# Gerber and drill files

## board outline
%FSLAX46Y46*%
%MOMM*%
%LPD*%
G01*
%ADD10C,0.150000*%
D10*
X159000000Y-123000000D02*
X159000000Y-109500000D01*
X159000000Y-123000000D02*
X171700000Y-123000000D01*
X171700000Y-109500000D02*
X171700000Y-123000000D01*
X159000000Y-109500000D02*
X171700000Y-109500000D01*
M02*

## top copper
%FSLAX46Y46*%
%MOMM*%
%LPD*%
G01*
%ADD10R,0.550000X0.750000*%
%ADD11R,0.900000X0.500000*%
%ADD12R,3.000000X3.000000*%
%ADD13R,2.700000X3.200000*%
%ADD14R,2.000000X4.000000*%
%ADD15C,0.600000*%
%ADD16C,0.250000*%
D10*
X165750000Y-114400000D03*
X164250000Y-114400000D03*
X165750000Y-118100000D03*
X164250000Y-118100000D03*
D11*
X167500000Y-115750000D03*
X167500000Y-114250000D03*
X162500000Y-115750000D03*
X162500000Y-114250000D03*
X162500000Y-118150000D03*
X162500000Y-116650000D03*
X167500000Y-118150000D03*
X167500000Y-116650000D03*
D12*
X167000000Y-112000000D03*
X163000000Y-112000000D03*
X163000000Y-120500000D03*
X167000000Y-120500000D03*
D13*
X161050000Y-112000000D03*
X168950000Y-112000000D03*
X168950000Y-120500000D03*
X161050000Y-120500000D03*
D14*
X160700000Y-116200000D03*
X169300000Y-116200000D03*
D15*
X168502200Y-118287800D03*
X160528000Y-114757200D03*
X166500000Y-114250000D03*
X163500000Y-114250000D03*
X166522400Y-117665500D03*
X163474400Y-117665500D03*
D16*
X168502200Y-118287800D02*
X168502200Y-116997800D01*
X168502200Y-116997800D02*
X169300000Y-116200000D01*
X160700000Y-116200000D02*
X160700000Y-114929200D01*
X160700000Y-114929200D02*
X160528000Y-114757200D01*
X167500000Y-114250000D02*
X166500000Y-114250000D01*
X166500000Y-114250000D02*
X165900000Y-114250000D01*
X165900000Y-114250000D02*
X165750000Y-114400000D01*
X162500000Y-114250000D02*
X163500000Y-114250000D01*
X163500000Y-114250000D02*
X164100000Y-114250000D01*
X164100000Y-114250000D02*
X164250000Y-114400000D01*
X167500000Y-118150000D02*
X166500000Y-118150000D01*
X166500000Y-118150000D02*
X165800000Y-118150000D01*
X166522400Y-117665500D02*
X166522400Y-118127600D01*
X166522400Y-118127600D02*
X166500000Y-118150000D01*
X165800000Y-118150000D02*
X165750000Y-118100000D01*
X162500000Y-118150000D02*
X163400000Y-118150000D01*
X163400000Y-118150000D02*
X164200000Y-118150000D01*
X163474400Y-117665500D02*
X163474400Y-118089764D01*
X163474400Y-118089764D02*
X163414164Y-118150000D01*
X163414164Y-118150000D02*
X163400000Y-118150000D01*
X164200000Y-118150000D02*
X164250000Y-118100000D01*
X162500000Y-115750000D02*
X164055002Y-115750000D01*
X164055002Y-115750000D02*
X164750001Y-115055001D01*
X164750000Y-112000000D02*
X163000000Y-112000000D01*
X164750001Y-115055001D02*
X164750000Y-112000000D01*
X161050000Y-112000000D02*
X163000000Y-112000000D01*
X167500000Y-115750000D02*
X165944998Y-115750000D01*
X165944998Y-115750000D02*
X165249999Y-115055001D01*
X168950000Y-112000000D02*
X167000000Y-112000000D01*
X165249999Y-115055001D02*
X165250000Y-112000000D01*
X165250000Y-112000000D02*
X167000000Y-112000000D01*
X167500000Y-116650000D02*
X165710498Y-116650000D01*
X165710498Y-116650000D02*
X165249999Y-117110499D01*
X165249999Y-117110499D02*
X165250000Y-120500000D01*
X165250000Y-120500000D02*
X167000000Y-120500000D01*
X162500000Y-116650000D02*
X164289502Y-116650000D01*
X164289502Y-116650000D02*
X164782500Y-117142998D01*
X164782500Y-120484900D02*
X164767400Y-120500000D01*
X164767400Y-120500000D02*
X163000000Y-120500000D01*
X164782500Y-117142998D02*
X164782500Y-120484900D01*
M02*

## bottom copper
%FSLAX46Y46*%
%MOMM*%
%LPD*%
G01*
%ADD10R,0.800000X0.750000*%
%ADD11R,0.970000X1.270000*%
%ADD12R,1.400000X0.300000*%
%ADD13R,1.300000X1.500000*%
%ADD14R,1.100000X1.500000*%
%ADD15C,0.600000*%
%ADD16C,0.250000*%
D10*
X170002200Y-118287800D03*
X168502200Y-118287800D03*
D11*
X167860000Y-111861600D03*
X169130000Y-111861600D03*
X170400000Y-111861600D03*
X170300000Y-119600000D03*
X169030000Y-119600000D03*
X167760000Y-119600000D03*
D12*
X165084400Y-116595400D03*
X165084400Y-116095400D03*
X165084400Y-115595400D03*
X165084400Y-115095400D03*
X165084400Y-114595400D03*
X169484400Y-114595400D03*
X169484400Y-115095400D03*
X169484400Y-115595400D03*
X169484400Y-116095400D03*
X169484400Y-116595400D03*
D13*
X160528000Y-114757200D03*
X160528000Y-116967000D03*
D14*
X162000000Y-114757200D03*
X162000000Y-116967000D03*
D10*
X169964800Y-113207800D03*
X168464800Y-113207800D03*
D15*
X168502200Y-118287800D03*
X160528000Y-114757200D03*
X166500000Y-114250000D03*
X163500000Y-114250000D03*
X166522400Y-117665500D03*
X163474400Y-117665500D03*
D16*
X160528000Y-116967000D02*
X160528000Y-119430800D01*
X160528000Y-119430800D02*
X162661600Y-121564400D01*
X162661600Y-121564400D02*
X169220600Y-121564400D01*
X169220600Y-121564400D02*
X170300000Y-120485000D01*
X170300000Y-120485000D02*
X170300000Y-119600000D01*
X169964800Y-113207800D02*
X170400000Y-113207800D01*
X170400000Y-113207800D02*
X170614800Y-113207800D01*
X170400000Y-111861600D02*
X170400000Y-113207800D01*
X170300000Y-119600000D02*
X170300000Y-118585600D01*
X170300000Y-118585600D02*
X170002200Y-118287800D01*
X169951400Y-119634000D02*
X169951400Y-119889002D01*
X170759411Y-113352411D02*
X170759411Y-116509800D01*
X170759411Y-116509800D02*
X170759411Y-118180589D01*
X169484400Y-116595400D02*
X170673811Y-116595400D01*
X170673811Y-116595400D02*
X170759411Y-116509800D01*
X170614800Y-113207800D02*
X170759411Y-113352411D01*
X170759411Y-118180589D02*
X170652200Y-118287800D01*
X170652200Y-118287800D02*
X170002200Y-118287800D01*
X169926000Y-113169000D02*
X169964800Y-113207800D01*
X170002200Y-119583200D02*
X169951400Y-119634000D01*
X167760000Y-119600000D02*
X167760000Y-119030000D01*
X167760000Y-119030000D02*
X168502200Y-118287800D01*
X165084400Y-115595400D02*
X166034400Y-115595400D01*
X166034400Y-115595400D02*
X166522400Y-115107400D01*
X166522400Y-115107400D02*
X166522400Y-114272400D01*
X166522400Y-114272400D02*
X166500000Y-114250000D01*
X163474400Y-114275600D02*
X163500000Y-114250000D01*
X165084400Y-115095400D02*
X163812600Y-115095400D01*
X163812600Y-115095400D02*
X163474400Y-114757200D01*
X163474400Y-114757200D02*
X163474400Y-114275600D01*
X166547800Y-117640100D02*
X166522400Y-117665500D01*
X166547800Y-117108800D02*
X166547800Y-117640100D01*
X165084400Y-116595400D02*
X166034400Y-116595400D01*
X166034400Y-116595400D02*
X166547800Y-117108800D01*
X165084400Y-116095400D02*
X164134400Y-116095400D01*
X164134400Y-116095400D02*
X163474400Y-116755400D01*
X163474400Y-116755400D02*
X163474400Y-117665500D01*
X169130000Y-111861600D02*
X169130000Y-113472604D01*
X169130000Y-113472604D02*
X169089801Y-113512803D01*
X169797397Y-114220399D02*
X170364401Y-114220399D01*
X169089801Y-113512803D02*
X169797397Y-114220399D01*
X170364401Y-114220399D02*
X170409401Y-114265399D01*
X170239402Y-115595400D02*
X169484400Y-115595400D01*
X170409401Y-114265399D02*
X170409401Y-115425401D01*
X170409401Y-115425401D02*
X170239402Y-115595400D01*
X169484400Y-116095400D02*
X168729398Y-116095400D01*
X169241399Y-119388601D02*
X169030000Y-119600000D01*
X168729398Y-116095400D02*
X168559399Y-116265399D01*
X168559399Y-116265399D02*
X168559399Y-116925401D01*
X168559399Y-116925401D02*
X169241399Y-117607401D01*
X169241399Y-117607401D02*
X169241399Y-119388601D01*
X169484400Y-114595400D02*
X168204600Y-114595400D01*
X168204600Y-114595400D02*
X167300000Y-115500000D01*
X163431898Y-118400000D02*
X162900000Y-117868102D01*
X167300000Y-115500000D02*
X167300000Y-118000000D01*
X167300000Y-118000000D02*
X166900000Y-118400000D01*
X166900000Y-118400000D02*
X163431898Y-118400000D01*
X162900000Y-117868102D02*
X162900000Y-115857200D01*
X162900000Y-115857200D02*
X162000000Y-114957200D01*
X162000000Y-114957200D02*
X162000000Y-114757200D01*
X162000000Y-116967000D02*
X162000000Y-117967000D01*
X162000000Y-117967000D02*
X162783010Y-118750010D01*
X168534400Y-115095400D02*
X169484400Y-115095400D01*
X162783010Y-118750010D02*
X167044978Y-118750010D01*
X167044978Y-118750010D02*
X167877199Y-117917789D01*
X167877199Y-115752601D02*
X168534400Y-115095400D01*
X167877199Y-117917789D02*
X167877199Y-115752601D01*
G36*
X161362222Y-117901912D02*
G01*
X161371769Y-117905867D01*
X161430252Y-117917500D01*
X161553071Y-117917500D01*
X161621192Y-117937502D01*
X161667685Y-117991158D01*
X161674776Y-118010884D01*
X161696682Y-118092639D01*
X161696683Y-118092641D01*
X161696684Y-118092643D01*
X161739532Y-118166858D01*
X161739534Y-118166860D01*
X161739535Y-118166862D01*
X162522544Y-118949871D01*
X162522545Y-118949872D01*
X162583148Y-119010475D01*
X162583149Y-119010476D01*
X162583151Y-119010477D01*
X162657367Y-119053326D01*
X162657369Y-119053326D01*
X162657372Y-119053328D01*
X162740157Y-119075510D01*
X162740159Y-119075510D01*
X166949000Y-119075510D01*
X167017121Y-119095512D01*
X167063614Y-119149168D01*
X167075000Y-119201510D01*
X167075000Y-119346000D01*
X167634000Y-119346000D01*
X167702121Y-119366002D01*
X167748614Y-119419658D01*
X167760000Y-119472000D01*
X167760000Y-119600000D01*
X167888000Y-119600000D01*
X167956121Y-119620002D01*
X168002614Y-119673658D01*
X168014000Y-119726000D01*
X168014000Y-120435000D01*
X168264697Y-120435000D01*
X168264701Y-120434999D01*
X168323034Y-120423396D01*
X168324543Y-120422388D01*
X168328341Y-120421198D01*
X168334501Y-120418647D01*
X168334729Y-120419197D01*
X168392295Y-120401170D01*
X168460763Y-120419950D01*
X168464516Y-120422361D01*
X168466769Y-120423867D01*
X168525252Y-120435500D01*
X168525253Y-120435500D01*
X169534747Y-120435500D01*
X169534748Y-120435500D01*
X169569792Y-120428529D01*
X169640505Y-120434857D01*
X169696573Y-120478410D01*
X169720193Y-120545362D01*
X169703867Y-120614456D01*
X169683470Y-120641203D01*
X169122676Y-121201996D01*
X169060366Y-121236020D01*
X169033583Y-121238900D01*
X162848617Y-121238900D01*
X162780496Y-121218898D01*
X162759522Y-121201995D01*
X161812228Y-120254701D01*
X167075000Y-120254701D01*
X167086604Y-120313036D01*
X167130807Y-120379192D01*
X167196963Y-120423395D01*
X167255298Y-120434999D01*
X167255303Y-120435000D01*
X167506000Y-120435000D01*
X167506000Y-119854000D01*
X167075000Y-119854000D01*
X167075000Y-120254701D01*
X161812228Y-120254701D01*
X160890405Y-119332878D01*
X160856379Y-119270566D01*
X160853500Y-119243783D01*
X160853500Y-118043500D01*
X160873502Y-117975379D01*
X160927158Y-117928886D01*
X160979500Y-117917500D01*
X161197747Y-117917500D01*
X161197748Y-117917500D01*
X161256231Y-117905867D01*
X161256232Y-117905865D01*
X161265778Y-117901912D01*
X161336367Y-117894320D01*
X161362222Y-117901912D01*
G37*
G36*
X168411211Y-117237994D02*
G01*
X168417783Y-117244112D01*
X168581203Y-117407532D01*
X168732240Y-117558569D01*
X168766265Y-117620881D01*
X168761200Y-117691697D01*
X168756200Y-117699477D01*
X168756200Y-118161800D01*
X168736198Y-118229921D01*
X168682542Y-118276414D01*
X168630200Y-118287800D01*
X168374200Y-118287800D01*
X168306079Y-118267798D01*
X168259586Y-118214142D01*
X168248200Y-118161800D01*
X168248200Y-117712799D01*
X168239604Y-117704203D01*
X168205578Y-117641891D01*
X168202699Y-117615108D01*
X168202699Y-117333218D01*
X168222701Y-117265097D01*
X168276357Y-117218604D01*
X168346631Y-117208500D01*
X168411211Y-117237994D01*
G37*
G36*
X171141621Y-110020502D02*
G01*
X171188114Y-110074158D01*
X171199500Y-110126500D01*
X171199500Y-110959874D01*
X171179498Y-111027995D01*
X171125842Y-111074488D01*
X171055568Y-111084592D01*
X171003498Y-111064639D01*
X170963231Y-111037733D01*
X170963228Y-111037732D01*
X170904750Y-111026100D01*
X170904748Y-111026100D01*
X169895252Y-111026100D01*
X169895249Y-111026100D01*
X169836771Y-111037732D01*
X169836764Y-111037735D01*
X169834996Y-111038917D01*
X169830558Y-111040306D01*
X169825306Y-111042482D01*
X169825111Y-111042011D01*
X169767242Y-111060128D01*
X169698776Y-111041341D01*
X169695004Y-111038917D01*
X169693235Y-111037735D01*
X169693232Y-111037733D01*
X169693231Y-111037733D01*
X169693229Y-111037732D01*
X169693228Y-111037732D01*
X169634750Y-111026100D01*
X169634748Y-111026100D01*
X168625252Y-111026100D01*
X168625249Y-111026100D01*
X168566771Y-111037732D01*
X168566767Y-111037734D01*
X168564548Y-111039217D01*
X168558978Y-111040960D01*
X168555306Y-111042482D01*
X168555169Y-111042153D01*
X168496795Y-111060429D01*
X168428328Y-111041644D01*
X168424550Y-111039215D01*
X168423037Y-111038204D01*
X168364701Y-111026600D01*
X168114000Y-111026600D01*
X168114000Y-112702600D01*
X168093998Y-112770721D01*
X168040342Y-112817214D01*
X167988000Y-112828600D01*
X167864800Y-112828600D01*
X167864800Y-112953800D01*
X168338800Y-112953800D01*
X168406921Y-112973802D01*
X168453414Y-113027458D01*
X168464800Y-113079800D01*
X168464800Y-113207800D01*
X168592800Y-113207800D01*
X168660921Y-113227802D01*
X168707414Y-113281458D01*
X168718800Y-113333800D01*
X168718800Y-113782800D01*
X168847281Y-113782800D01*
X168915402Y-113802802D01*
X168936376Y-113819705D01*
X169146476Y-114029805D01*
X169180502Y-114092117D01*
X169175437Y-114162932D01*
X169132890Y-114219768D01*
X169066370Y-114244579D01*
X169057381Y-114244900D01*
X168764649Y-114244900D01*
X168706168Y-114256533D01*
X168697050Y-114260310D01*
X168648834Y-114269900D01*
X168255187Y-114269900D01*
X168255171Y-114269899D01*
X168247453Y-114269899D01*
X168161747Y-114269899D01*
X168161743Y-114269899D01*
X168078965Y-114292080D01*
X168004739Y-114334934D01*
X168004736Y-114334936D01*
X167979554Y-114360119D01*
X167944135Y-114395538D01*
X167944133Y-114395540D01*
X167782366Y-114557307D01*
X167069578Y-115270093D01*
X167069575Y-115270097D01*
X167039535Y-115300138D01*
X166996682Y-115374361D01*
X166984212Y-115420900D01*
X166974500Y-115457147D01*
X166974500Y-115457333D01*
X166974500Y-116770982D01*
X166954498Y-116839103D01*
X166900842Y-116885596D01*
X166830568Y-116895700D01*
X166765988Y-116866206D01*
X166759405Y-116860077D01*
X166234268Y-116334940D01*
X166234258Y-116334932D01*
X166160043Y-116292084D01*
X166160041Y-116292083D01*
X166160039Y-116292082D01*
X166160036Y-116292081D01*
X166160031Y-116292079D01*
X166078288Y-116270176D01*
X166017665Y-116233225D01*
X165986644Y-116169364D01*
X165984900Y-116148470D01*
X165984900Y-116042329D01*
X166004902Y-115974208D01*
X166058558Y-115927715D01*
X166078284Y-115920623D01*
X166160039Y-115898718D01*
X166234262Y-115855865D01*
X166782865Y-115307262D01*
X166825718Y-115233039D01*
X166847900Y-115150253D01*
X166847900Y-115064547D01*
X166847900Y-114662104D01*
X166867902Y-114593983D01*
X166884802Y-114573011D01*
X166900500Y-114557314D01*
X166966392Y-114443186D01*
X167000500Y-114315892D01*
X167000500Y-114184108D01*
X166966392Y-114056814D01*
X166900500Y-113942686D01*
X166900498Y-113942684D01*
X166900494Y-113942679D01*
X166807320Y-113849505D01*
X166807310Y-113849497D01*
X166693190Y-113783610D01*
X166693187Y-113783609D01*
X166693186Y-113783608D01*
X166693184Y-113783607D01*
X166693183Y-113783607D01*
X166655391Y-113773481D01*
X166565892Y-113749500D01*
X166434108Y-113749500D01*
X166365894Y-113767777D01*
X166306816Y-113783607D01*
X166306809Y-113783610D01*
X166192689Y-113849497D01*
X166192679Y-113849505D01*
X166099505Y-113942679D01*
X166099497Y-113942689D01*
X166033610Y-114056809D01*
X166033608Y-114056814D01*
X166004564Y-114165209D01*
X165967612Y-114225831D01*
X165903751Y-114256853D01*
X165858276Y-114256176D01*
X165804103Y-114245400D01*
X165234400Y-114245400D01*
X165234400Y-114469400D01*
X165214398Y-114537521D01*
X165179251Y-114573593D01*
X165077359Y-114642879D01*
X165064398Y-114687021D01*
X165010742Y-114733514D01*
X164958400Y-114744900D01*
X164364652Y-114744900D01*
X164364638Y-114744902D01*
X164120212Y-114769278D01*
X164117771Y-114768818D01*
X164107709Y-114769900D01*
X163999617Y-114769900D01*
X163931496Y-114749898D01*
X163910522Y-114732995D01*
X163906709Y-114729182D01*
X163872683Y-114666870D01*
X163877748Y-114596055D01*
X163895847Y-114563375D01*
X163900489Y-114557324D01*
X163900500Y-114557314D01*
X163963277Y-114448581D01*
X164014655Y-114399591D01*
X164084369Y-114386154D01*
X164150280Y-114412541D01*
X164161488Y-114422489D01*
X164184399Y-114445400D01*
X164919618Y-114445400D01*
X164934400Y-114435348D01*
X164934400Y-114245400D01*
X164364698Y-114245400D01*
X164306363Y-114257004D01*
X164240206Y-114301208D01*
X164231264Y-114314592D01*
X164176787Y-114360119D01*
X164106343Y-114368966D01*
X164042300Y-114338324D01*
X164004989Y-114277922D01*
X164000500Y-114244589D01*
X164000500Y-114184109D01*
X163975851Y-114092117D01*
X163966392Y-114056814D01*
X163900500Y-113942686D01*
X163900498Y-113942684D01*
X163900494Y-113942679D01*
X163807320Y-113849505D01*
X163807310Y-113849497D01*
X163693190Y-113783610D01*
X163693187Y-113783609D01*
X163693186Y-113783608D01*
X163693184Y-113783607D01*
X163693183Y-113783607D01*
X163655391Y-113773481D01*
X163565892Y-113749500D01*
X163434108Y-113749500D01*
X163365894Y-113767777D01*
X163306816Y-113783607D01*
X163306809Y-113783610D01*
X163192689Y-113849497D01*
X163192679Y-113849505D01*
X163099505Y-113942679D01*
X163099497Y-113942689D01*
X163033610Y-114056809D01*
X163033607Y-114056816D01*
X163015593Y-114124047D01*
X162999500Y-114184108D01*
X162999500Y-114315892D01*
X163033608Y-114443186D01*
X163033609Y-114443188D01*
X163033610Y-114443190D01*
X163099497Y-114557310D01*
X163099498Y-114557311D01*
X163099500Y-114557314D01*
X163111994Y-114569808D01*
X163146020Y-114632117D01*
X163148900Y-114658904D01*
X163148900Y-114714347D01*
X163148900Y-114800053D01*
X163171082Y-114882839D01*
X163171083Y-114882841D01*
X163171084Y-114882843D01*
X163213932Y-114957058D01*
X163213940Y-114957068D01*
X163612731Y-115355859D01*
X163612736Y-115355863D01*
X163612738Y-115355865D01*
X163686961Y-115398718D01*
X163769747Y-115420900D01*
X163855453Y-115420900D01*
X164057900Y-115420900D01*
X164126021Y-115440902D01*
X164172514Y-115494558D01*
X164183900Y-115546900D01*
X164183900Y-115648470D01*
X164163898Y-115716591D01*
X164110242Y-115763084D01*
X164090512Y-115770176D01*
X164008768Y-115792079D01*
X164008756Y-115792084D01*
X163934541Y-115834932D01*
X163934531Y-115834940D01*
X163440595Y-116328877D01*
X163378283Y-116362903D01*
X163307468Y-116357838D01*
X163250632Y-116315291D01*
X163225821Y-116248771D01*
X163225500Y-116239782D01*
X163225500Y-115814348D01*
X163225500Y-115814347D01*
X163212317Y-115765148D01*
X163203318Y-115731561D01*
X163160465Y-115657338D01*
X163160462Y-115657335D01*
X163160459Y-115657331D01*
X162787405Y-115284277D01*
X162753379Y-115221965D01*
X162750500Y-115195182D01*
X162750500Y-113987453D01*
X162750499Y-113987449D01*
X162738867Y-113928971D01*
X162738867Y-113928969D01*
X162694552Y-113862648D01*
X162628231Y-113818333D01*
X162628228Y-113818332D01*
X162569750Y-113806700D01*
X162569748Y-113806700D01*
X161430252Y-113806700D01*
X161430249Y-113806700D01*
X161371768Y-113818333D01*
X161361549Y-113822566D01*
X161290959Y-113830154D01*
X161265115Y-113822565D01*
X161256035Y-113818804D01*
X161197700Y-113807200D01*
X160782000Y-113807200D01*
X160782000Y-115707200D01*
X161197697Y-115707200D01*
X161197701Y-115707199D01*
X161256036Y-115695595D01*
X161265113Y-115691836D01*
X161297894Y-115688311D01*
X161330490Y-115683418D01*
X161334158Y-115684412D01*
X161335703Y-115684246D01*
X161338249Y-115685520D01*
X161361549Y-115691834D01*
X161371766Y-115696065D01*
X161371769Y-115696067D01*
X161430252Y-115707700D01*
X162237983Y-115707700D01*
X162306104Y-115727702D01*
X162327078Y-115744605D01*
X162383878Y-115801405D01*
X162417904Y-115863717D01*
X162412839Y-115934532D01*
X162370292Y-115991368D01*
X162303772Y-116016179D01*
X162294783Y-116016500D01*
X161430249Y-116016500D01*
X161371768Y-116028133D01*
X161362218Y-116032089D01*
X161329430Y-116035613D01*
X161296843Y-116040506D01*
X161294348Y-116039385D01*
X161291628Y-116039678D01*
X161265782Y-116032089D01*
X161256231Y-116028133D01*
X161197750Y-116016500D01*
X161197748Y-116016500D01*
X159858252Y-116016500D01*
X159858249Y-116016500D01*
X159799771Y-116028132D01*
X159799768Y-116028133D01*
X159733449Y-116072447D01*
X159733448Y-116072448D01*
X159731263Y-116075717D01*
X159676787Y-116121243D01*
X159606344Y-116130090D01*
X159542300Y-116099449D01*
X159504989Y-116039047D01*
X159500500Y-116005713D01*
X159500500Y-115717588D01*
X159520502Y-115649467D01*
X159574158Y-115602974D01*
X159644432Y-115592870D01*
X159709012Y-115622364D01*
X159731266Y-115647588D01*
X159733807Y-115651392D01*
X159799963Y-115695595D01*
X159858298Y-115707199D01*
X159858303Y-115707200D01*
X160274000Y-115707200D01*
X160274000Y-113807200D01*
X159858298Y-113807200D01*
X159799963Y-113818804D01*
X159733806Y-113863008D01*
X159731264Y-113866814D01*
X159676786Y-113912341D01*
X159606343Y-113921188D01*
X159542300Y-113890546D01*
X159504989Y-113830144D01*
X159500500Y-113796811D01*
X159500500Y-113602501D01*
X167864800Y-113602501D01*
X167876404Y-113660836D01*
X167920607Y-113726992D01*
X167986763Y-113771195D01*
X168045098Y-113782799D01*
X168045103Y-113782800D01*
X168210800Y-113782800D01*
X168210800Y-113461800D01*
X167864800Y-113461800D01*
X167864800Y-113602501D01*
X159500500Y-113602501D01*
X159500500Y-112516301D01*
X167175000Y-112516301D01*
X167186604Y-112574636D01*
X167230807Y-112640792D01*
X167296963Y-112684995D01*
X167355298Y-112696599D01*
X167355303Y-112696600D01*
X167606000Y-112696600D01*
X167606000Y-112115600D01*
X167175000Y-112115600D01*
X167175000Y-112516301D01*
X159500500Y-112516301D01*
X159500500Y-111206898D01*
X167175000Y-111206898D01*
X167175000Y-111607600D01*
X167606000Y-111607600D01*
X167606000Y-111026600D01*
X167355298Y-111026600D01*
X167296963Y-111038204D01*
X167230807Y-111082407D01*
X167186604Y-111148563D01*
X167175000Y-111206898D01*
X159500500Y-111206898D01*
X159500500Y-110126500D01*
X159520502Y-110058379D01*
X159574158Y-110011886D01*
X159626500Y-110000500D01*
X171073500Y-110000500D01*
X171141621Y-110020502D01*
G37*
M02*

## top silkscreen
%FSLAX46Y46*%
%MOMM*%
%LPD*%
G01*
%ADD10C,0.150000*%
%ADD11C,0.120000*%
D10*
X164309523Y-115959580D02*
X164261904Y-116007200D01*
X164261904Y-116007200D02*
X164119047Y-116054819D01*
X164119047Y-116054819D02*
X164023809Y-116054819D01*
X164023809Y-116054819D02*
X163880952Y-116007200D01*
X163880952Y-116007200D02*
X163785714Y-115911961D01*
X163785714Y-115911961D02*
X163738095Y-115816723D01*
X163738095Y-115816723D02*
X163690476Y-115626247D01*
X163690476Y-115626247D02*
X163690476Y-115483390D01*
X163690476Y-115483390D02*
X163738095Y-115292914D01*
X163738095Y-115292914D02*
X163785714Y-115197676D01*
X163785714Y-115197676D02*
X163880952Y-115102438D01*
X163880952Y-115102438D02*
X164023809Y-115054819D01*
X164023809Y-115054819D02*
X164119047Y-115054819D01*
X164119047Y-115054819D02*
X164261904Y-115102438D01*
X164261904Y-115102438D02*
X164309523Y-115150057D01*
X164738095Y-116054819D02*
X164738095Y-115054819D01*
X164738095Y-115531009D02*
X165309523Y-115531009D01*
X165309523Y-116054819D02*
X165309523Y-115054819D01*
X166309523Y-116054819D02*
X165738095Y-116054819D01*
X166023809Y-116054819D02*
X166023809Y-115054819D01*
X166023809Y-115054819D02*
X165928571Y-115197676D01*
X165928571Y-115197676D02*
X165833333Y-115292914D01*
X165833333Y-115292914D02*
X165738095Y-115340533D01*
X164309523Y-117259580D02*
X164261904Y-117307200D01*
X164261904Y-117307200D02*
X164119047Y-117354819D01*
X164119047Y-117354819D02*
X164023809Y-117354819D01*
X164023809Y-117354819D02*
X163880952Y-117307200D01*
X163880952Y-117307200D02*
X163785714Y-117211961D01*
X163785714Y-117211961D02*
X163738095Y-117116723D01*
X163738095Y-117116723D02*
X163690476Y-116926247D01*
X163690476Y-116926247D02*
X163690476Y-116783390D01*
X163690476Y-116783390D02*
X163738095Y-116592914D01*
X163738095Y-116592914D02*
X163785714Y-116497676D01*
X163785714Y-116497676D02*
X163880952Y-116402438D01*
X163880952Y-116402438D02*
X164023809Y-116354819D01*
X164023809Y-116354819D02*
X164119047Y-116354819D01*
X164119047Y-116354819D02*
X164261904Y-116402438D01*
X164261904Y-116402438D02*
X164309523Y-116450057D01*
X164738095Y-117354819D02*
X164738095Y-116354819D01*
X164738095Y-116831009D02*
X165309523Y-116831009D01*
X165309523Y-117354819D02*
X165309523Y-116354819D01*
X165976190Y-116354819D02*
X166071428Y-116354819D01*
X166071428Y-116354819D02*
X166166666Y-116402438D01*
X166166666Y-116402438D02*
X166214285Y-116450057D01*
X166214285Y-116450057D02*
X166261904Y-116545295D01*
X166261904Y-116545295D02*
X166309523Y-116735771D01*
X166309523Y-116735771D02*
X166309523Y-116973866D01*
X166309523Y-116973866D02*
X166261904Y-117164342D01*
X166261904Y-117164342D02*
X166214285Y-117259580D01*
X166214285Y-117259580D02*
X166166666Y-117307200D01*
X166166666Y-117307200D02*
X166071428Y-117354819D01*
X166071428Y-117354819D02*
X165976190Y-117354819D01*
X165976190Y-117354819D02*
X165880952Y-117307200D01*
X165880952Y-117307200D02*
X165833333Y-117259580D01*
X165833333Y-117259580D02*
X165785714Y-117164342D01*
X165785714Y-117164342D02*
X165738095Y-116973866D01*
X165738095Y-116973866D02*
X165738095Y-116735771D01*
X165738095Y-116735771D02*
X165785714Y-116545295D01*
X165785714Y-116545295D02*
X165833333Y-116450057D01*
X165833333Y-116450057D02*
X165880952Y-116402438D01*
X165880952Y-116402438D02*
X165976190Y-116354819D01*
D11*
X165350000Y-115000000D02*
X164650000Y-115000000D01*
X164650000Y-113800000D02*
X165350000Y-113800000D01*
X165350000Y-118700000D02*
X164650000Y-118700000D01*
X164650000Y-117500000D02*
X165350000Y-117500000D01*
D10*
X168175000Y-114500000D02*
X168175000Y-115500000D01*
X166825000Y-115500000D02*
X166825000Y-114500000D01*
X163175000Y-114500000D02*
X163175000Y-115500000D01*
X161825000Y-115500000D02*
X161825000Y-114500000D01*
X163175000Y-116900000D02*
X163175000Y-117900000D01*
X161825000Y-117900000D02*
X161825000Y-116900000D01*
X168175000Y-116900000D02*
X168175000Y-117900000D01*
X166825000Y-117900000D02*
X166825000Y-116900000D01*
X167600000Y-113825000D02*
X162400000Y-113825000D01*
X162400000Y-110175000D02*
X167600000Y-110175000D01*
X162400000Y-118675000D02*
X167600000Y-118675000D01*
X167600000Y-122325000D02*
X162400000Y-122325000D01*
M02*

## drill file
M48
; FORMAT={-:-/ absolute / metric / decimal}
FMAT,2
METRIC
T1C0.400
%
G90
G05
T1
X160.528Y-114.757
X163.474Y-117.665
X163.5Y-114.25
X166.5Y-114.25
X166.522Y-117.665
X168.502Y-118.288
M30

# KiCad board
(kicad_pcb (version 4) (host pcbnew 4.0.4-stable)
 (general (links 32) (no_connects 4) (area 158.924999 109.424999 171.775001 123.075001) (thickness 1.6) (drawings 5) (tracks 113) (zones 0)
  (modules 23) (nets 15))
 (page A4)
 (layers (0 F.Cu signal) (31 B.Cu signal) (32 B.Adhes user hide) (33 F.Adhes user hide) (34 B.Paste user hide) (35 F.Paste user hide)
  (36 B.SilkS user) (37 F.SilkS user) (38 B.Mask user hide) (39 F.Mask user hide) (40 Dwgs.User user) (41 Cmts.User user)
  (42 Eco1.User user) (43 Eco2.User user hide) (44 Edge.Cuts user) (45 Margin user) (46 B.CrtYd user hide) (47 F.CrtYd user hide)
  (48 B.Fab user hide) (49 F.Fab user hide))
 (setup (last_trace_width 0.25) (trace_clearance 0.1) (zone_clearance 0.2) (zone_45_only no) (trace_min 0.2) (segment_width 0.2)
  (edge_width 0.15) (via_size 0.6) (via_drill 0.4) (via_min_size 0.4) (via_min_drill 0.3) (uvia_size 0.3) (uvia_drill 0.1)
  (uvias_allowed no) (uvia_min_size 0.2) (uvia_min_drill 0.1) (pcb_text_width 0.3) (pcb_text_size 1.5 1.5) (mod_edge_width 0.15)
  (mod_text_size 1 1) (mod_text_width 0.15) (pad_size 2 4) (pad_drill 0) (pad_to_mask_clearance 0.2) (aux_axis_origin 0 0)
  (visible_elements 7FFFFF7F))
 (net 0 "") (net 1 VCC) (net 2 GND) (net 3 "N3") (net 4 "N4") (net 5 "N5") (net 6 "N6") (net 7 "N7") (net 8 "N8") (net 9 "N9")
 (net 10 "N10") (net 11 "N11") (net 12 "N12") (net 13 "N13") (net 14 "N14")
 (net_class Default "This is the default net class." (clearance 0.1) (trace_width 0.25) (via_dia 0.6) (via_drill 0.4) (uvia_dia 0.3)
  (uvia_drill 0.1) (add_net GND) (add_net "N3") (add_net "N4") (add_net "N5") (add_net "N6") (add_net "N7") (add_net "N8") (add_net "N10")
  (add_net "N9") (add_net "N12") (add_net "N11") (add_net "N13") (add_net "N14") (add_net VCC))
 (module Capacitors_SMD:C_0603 (layer B.Cu) (at 169.2522 118.2878 180)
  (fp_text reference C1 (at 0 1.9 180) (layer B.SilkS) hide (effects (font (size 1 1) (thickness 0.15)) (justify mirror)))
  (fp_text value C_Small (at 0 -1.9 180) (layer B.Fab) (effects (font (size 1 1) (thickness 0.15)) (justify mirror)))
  (pad 1 smd rect (at -0.75 0 180) (size 0.8 0.75) (layers B.Cu B.Paste B.Mask) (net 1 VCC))
  (pad 2 smd rect (at 0.75 0 180) (size 0.8 0.75) (layers B.Cu B.Paste B.Mask) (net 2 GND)))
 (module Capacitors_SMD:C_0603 (layer F.Cu) (at 165 114.4 180)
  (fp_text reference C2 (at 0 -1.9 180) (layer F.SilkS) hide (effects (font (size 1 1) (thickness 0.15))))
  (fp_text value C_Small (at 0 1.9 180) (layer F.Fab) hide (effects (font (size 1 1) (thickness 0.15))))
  (fp_line (start -0.35 -0.6) (end 0.35 -0.6) (layer F.SilkS) (width 0.12))
  (fp_line (start 0.35 0.6) (end -0.35 0.6) (layer F.SilkS) (width 0.12))
  (pad 1 smd rect (at -0.75 0 180) (size 0.55 0.75) (layers F.Cu F.Paste F.Mask) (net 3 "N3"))
  (pad 2 smd rect (at 0.75 0 180) (size 0.55 0.75) (layers F.Cu F.Paste F.Mask) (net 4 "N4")))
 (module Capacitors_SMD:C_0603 (layer F.Cu) (at 165 118.1 180)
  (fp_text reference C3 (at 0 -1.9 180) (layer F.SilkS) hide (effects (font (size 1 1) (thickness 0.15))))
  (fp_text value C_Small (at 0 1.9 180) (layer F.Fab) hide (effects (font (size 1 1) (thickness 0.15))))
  (fp_line (start -0.35 -0.6) (end 0.35 -0.6) (layer F.SilkS) (width 0.12))
  (fp_line (start 0.35 0.6) (end -0.35 0.6) (layer F.SilkS) (width 0.12))
  (pad 1 smd rect (at -0.75 0 180) (size 0.55 0.75) (layers F.Cu F.Paste F.Mask) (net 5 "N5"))
  (pad 2 smd rect (at 0.75 0 180) (size 0.55 0.75) (layers F.Cu F.Paste F.Mask) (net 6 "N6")))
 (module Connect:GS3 (layer B.Cu) (at 169.13 111.8616 270)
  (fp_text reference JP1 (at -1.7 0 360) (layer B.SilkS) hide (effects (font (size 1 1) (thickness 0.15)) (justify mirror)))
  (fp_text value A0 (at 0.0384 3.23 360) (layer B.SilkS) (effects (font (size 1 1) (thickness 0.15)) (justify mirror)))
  (pad 1 smd rect (at 0 1.27 270) (size 1.27 0.97) (layers B.Cu B.Paste B.Mask) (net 2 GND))
  (pad 2 smd rect (at 0 0 270) (size 1.27 0.97) (layers B.Cu B.Paste B.Mask) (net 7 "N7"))
  (pad 3 smd rect (at 0 -1.27 270) (size 1.27 0.97) (layers B.Cu B.Paste B.Mask) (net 1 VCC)))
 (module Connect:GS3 (layer B.Cu) (at 169.03 119.6 90)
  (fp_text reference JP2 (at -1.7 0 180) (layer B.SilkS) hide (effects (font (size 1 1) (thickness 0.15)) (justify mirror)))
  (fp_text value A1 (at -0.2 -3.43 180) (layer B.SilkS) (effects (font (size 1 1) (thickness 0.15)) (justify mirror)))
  (pad 1 smd rect (at 0 1.27 90) (size 1.27 0.97) (layers B.Cu B.Paste B.Mask) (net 1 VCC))
  (pad 2 smd rect (at 0 0 90) (size 1.27 0.97) (layers B.Cu B.Paste B.Mask) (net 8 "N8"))
  (pad 3 smd rect (at 0 -1.27 90) (size 1.27 0.97) (layers B.Cu B.Paste B.Mask) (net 2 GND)))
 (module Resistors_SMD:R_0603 (layer F.Cu) (at 167.5 115 90)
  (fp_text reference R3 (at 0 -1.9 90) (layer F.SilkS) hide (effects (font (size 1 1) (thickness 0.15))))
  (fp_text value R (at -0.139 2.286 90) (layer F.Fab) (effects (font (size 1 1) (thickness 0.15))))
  (fp_line (start 0.5 0.675) (end -0.5 0.675) (layer F.SilkS) (width 0.15))
  (fp_line (start -0.5 -0.675) (end 0.5 -0.675) (layer F.SilkS) (width 0.15))
  (pad 1 smd rect (at -0.75 0 90) (size 0.5 0.9) (layers F.Cu F.Paste F.Mask) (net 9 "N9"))
  (pad 2 smd rect (at 0.75 0 90) (size 0.5 0.9) (layers F.Cu F.Paste F.Mask) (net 3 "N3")))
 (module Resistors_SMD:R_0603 (layer F.Cu) (at 162.5 115 90)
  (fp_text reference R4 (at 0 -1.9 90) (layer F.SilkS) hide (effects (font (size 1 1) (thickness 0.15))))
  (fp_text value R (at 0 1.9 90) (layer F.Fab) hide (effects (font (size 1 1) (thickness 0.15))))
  (fp_line (start 0.5 0.675) (end -0.5 0.675) (layer F.SilkS) (width 0.15))
  (fp_line (start -0.5 -0.675) (end 0.5 -0.675) (layer F.SilkS) (width 0.15))
  (pad 1 smd rect (at -0.75 0 90) (size 0.5 0.9) (layers F.Cu F.Paste F.Mask) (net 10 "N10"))
  (pad 2 smd rect (at 0.75 0 90) (size 0.5 0.9) (layers F.Cu F.Paste F.Mask) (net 4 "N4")))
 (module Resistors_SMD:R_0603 (layer F.Cu) (at 162.5 117.4 90)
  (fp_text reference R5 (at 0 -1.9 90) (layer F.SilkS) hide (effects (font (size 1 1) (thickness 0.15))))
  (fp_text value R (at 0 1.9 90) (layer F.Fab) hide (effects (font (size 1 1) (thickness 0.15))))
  (fp_line (start 0.5 0.675) (end -0.5 0.675) (layer F.SilkS) (width 0.15))
  (fp_line (start -0.5 -0.675) (end 0.5 -0.675) (layer F.SilkS) (width 0.15))
  (pad 1 smd rect (at -0.75 0 90) (size 0.5 0.9) (layers F.Cu F.Paste F.Mask) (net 6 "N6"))
  (pad 2 smd rect (at 0.75 0 90) (size 0.5 0.9) (layers F.Cu F.Paste F.Mask) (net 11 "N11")))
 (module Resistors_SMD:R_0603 (layer F.Cu) (at 167.5 117.4 90)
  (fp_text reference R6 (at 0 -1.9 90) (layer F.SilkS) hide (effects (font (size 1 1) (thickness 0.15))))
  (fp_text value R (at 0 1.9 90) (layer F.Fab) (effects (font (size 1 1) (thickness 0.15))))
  (fp_line (start 0.5 0.675) (end -0.5 0.675) (layer F.SilkS) (width 0.15))
  (fp_line (start -0.5 -0.675) (end 0.5 -0.675) (layer F.SilkS) (width 0.15))
  (pad 1 smd rect (at -0.75 0 90) (size 0.5 0.9) (layers F.Cu F.Paste F.Mask) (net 5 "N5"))
  (pad 2 smd rect (at 0.75 0 90) (size 0.5 0.9) (layers F.Cu F.Paste F.Mask) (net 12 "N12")))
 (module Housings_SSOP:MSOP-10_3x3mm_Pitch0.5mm (layer B.Cu) (at 167.2844 115.5954)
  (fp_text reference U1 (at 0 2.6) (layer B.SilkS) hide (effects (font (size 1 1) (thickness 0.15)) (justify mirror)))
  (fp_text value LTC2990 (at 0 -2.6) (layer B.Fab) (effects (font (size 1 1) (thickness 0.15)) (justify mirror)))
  (pad 1 smd rect (at -2.2 1) (size 1.4 0.3) (layers B.Cu B.Paste B.Mask) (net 5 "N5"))
  (pad 2 smd rect (at -2.2 0.5) (size 1.4 0.3) (layers B.Cu B.Paste B.Mask) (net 6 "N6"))
  (pad 3 smd rect (at -2.2 0) (size 1.4 0.3) (layers B.Cu B.Paste B.Mask) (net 3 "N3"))
  (pad 4 smd rect (at -2.2 -0.5) (size 1.4 0.3) (layers B.Cu B.Paste B.Mask) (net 4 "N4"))
  (pad 5 smd rect (at -2.2 -1) (size 1.4 0.3) (layers B.Cu B.Paste B.Mask) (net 2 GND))
  (pad 6 smd rect (at 2.2 -1) (size 1.4 0.3) (layers B.Cu B.Paste B.Mask) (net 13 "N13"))
  (pad 7 smd rect (at 2.2 -0.5) (size 1.4 0.3) (layers B.Cu B.Paste B.Mask) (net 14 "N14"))
  (pad 8 smd rect (at 2.2 0) (size 1.4 0.3) (layers B.Cu B.Paste B.Mask) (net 7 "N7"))
  (pad 9 smd rect (at 2.2 0.5) (size 1.4 0.3) (layers B.Cu B.Paste B.Mask) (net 8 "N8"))
  (pad 10 smd rect (at 2.2 1) (size 1.4 0.3) (layers B.Cu B.Paste B.Mask) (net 1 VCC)))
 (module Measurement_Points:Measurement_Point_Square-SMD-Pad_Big (layer F.Cu) (at 167 112)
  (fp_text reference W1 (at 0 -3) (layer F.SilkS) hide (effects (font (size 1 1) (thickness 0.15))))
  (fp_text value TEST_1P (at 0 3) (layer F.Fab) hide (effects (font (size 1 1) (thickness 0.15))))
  (pad 1 smd rect (at 0 0) (size 3 3) (layers F.Cu F.Mask) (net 9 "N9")))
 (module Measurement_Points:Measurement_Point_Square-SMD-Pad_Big (layer F.Cu) (at 163 112)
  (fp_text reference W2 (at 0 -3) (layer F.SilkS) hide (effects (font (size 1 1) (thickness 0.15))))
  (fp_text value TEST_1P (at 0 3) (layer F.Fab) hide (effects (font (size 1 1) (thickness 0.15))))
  (pad 1 smd rect (at 0 0) (size 3 3) (layers F.Cu F.Mask) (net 10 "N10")))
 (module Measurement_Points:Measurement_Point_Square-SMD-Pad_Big (layer F.Cu) (at 163 120.5 180)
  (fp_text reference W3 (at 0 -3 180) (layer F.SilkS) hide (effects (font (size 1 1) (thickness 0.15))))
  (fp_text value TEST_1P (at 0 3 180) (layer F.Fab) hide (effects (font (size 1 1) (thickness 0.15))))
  (pad 1 smd rect (at 0 0 180) (size 3 3) (layers F.Cu F.Mask) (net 11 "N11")))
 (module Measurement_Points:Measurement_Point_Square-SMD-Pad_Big (layer F.Cu) (at 167 120.5 180)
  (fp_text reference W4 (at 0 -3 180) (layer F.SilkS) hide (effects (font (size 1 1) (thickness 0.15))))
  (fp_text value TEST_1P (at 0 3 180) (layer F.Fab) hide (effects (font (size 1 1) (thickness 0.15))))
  (pad 1 smd rect (at 0 0 180) (size 3 3) (layers F.Cu F.Mask) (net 12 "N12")))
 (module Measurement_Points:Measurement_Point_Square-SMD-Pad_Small (layer B.Cu) (at 160.528 114.7572 180)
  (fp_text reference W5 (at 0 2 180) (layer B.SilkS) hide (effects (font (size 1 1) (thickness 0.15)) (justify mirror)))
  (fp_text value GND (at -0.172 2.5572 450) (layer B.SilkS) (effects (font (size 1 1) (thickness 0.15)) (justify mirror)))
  (pad 1 smd rect (at 0 0 180) (size 1.3 1.5) (layers B.Cu B.Mask) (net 2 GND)))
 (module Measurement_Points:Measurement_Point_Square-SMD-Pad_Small (layer B.Cu) (at 160.528 116.967 180)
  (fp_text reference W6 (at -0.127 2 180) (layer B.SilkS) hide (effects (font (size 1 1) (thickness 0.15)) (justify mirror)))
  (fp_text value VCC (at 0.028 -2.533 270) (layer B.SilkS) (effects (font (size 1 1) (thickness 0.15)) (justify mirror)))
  (pad 1 smd rect (at 0 0 180) (size 1.3 1.5) (layers B.Cu B.Mask) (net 1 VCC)))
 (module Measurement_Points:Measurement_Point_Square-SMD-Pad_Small (layer B.Cu) (at 162 114.7572)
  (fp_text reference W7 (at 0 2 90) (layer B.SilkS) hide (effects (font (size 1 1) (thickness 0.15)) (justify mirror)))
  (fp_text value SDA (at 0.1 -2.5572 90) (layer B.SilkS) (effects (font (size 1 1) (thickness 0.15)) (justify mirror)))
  (pad 1 smd rect (at 0 0) (size 1.1 1.5) (layers B.Cu B.Mask) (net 13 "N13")))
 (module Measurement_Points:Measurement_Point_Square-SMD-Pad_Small (layer B.Cu) (at 162 116.967)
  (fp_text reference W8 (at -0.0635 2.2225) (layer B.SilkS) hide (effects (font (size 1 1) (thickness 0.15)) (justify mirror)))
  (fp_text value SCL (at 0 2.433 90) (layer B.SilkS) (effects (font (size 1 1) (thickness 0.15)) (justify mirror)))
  (pad 1 smd rect (at 0 0) (size 1.1 1.5) (layers B.Cu B.Mask) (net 14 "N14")))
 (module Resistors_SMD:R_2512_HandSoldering (layer F.Cu) (at 165 112)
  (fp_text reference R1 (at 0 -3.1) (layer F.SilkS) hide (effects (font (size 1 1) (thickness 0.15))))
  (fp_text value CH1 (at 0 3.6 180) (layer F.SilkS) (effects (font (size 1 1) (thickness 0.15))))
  (fp_line (start 2.6 1.825) (end -2.6 1.825) (layer F.SilkS) (width 0.15))
  (fp_line (start -2.6 -1.825) (end 2.6 -1.825) (layer F.SilkS) (width 0.15))
  (pad 1 smd rect (at -3.95 0) (size 2.7 3.2) (layers F.Cu F.Paste F.Mask) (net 10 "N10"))
  (pad 2 smd rect (at 3.95 0) (size 2.7 3.2) (layers F.Cu F.Paste F.Mask) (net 9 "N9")))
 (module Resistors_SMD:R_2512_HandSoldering (layer F.Cu) (at 165 120.5 180)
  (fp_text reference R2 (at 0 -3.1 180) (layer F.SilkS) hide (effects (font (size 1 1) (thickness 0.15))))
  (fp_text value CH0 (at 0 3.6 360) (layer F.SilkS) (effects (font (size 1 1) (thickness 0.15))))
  (fp_line (start 2.6 1.825) (end -2.6 1.825) (layer F.SilkS) (width 0.15))
  (fp_line (start -2.6 -1.825) (end 2.6 -1.825) (layer F.SilkS) (width 0.15))
  (pad 1 smd rect (at -3.95 0 180) (size 2.7 3.2) (layers F.Cu F.Paste F.Mask) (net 12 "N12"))
  (pad 2 smd rect (at 3.95 0 180) (size 2.7 3.2) (layers F.Cu F.Paste F.Mask) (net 11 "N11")))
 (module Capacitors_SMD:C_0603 (layer B.Cu) (at 169.2148 113.2078 180)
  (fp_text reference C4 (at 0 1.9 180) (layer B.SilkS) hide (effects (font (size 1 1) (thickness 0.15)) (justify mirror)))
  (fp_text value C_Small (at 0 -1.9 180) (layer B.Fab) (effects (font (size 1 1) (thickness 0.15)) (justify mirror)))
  (pad 1 smd rect (at -0.75 0 180) (size 0.8 0.75) (layers B.Cu B.Paste B.Mask) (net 1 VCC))
  (pad 2 smd rect (at 0.75 0 180) (size 0.8 0.75) (layers B.Cu B.Paste B.Mask) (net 2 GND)))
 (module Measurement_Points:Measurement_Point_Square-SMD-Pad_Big (layer F.Cu) (at 160.7 116.2)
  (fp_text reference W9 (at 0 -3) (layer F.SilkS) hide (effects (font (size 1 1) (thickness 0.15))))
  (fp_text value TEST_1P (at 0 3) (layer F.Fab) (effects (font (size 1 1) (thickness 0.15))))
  (pad 1 smd rect (at 0 0) (size 2 4) (layers F.Cu F.Mask) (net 2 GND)))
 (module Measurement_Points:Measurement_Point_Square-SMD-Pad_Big (layer F.Cu) (at 169.3 116.2)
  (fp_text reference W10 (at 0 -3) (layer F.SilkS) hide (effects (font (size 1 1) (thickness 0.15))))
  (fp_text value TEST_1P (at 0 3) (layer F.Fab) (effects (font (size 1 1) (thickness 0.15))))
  (pad 1 smd rect (at 0 0) (size 2 4) (layers F.Cu F.Mask) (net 2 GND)))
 (gr_line (start 159 123) (end 159 109.5) (layer Edge.Cuts) (width 0.15))
 (gr_line (start 159 123) (end 171.7 123) (layer Edge.Cuts) (width 0.15))
 (gr_line (start 171.7 109.5) (end 171.7 123) (layer Edge.Cuts) (width 0.15))
 (gr_line (start 159 109.5) (end 171.7 109.5) (layer Edge.Cuts) (width 0.15))
 (segment (start 160.528 116.967) (end 160.528 119.4308) (width 0.25) (layer B.Cu) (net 1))
 (segment (start 160.528 119.4308) (end 162.6616 121.5644) (width 0.25) (layer B.Cu) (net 1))
 (segment (start 162.6616 121.5644) (end 169.2206 121.5644) (width 0.25) (layer B.Cu) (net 1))
 (segment (start 169.2206 121.5644) (end 170.3 120.485) (width 0.25) (layer B.Cu) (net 1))
 (segment (start 170.3 120.485) (end 170.3 119.6) (width 0.25) (layer B.Cu) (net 1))
 (segment (start 169.9648 113.2078) (end 170.4 113.2078) (width 0.25) (layer B.Cu) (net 1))
 (segment (start 170.4 113.2078) (end 170.6148 113.2078) (width 0.25) (layer B.Cu) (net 1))
 (segment (start 170.4 111.8616) (end 170.4 113.2078) (width 0.25) (layer B.Cu) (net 1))
 (segment (start 170.3 119.6) (end 170.3 118.5856) (width 0.25) (layer B.Cu) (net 1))
 (segment (start 170.3 118.5856) (end 170.0022 118.2878) (width 0.25) (layer B.Cu) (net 1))
 (segment (start 169.9514 119.634) (end 169.9514 119.889002) (width 0.25) (layer B.Cu) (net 1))
 (segment (start 170.759411 113.352411) (end 170.759411 116.5098) (width 0.25) (layer B.Cu) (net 1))
 (segment (start 170.759411 116.5098) (end 170.759411 118.180589) (width 0.25) (layer B.Cu) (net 1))
 (segment (start 169.4844 116.5954) (end 170.673811 116.5954) (width 0.25) (layer B.Cu) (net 1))
 (segment (start 170.673811 116.5954) (end 170.759411 116.5098) (width 0.25) (layer B.Cu) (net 1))
 (segment (start 170.6148 113.2078) (end 170.759411 113.352411) (width 0.25) (layer B.Cu) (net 1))
 (segment (start 170.759411 118.180589) (end 170.6522 118.2878) (width 0.25) (layer B.Cu) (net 1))
 (segment (start 170.6522 118.2878) (end 170.0022 118.2878) (width 0.25) (layer B.Cu) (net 1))
 (segment (start 169.926 113.169) (end 169.9648 113.2078) (width 0.25) (layer B.Cu) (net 1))
 (segment (start 170.0022 119.5832) (end 169.9514 119.634) (width 0.25) (layer B.Cu) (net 1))
 (segment (start 168.5022 118.2878) (end 168.5022 116.9978) (width 0.25) (layer F.Cu) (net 2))
 (segment (start 168.5022 116.9978) (end 169.3 116.2) (width 0.25) (layer F.Cu) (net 2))
 (via (at 168.5022 118.2878) (size 0.6) (drill 0.4) (layers F.Cu B.Cu) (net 2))
 (segment (start 160.7 116.2) (end 160.7 114.9292) (width 0.25) (layer F.Cu) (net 2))
 (segment (start 160.7 114.9292) (end 160.528 114.7572) (width 0.25) (layer F.Cu) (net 2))
 (via (at 160.528 114.7572) (size 0.6) (drill 0.4) (layers F.Cu B.Cu) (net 2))
 (segment (start 167.76 119.6) (end 167.76 119.03) (width 0.25) (layer B.Cu) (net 2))
 (segment (start 167.76 119.03) (end 168.5022 118.2878) (width 0.25) (layer B.Cu) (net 2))
 (segment (start 167.5 114.25) (end 166.5 114.25) (width 0.25) (layer F.Cu) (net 3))
 (segment (start 166.5 114.25) (end 165.9 114.25) (width 0.25) (layer F.Cu) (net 3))
 (via (at 166.5 114.25) (size 0.6) (drill 0.4) (layers F.Cu B.Cu) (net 3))
 (segment (start 165.0844 115.5954) (end 166.0344 115.5954) (width 0.25) (layer B.Cu) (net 3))
 (segment (start 166.0344 115.5954) (end 166.5224 115.1074) (width 0.25) (layer B.Cu) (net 3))
 (segment (start 166.5224 115.1074) (end 166.5224 114.2724) (width 0.25) (layer B.Cu) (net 3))
 (segment (start 166.5224 114.2724) (end 166.5 114.25) (width 0.25) (layer B.Cu) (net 3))
 (segment (start 165.9 114.25) (end 165.75 114.4) (width 0.25) (layer F.Cu) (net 3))
 (segment (start 162.5 114.25) (end 163.5 114.25) (width 0.25) (layer F.Cu) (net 4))
 (segment (start 163.5 114.25) (end 164.1 114.25) (width 0.25) (layer F.Cu) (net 4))
 (via (at 163.5 114.25) (size 0.6) (drill 0.4) (layers F.Cu B.Cu) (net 4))
 (segment (start 163.4744 114.2756) (end 163.5 114.25) (width 0.25) (layer B.Cu) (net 4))
 (segment (start 165.0844 115.0954) (end 163.8126 115.0954) (width 0.25) (layer B.Cu) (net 4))
 (segment (start 163.8126 115.0954) (end 163.4744 114.7572) (width 0.25) (layer B.Cu) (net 4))
 (segment (start 163.4744 114.7572) (end 163.4744 114.2756) (width 0.25) (layer B.Cu) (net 4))
 (segment (start 164.1 114.25) (end 164.25 114.4) (width 0.25) (layer F.Cu) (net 4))
 (segment (start 167.5 118.15) (end 166.5 118.15) (width 0.25) (layer F.Cu) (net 5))
 (segment (start 166.5 118.15) (end 165.8 118.15) (width 0.25) (layer F.Cu) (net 5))
 (segment (start 166.5224 117.6655) (end 166.5224 118.1276) (width 0.25) (layer F.Cu) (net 5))
 (segment (start 166.5224 118.1276) (end 166.5 118.15) (width 0.25) (layer F.Cu) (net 5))
 (segment (start 166.5478 117.6401) (end 166.5224 117.6655) (width 0.25) (layer B.Cu) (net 5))
 (via (at 166.5224 117.6655) (size 0.6) (drill 0.4) (layers F.Cu B.Cu) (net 5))
 (segment (start 165.8 118.15) (end 165.75 118.1) (width 0.25) (layer F.Cu) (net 5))
 (segment (start 166.5478 117.1088) (end 166.5478 117.6401) (width 0.25) (layer B.Cu) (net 5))
 (segment (start 165.0844 116.5954) (end 166.0344 116.5954) (width 0.25) (layer B.Cu) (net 5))
 (segment (start 166.0344 116.5954) (end 166.5478 117.1088) (width 0.25) (layer B.Cu) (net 5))
 (segment (start 162.5 118.15) (end 163.4 118.15) (width 0.25) (layer F.Cu) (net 6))
 (segment (start 163.4 118.15) (end 164.2 118.15) (width 0.25) (layer F.Cu) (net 6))
 (segment (start 163.4744 117.6655) (end 163.4744 118.089764) (width 0.25) (layer F.Cu) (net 6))
 (segment (start 163.4744 118.089764) (end 163.414164 118.15) (width 0.25) (layer F.Cu) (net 6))
 (segment (start 163.414164 118.15) (end 163.4 118.15) (width 0.25) (layer F.Cu) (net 6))
 (via (at 163.4744 117.6655) (size 0.6) (drill 0.4) (layers F.Cu B.Cu) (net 6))
 (segment (start 164.2 118.15) (end 164.25 118.1) (width 0.25) (layer F.Cu) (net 6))
 (segment (start 165.0844 116.0954) (end 164.1344 116.0954) (width 0.25) (layer B.Cu) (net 6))
 (segment (start 164.1344 116.0954) (end 163.4744 116.7554) (width 0.25) (layer B.Cu) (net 6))
 (segment (start 163.4744 116.7554) (end 163.4744 117.6655) (width 0.25) (layer B.Cu) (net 6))
 (segment (start 169.13 111.8616) (end 169.13 113.472604) (width 0.25) (layer B.Cu) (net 7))
 (segment (start 169.13 113.472604) (end 169.089801 113.512803) (width 0.25) (layer B.Cu) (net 7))
 (segment (start 169.797397 114.220399) (end 170.364401 114.220399) (width 0.25) (layer B.Cu) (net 7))
 (segment (start 169.089801 113.512803) (end 169.797397 114.220399) (width 0.25) (layer B.Cu) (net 7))
 (segment (start 170.364401 114.220399) (end 170.409401 114.265399) (width 0.25) (layer B.Cu) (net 7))
 (segment (start 170.239402 115.5954) (end 169.4844 115.5954) (width 0.25) (layer B.Cu) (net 7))
 (segment (start 170.409401 114.265399) (end 170.409401 115.425401) (width 0.25) (layer B.Cu) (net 7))
 (segment (start 170.409401 115.425401) (end 170.239402 115.5954) (width 0.25) (layer B.Cu) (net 7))
 (segment (start 169.4844 116.0954) (end 168.729398 116.0954) (width 0.25) (layer B.Cu) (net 8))
 (segment (start 169.241399 119.388601) (end 169.03 119.6) (width 0.25) (layer B.Cu) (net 8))
 (segment (start 168.729398 116.0954) (end 168.559399 116.265399) (width 0.25) (layer B.Cu) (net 8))
 (segment (start 168.559399 116.265399) (end 168.559399 116.925401) (width 0.25) (layer B.Cu) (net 8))
 (segment (start 168.559399 116.925401) (end 169.241399 117.607401) (width 0.25) (layer B.Cu) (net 8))
 (segment (start 169.241399 117.607401) (end 169.241399 119.388601) (width 0.25) (layer B.Cu) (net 8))
 (segment (start 162.5 115.75) (end 164.055002 115.75) (width 0.25) (layer F.Cu) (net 10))
 (segment (start 164.055002 115.75) (end 164.750001 115.055001) (width 0.25) (layer F.Cu) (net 10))
 (segment (start 164.75 112) (end 163 112) (width 0.25) (layer F.Cu) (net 10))
 (segment (start 164.750001 115.055001) (end 164.75 112) (width 0.25) (layer F.Cu) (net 10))
 (segment (start 161.05 112) (end 163 112) (width 0.25) (layer F.Cu) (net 10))
 (segment (start 167.5 115.75) (end 165.944998 115.75) (width 0.25) (layer F.Cu) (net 9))
 (segment (start 165.944998 115.75) (end 165.249999 115.055001) (width 0.25) (layer F.Cu) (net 9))
 (segment (start 168.95 112) (end 167 112) (width 0.25) (layer F.Cu) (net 9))
 (segment (start 165.249999 115.055001) (end 165.25 112) (width 0.25) (layer F.Cu) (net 9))
 (segment (start 165.25 112) (end 167 112) (width 0.25) (layer F.Cu) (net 9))
 (segment (start 167.5 116.65) (end 165.710498 116.65) (width 0.25) (layer F.Cu) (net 12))
 (segment (start 165.710498 116.65) (end 165.249999 117.110499) (width 0.25) (layer F.Cu) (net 12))
 (segment (start 165.249999 117.110499) (end 165.25 120.5) (width 0.25) (layer F.Cu) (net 12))
 (segment (start 165.25 120.5) (end 167 120.5) (width 0.25) (layer F.Cu) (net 12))
 (segment (start 162.5 116.65) (end 164.289502 116.65) (width 0.25) (layer F.Cu) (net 11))
 (segment (start 164.289502 116.65) (end 164.7825 117.142998) (width 0.25) (layer F.Cu) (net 11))
 (segment (start 164.7825 120.4849) (end 164.7674 120.5) (width 0.25) (layer F.Cu) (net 11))
 (segment (start 164.7674 120.5) (end 163 120.5) (width 0.25) (layer F.Cu) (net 11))
 (segment (start 164.7825 117.142998) (end 164.7825 120.4849) (width 0.25) (layer F.Cu) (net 11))
 (segment (start 169.4844 114.5954) (end 168.2046 114.5954) (width 0.25) (layer B.Cu) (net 13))
 (segment (start 168.2046 114.5954) (end 167.3 115.5) (width 0.25) (layer B.Cu) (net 13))
 (segment (start 163.431898 118.4) (end 162.9 117.868102) (width 0.25) (layer B.Cu) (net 13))
 (segment (start 167.3 115.5) (end 167.3 118) (width 0.25) (layer B.Cu) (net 13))
 (segment (start 167.3 118) (end 166.9 118.4) (width 0.25) (layer B.Cu) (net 13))
 (segment (start 166.9 118.4) (end 163.431898 118.4) (width 0.25) (layer B.Cu) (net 13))
 (segment (start 162.9 117.868102) (end 162.9 115.8572) (width 0.25) (layer B.Cu) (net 13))
 (segment (start 162.9 115.8572) (end 162 114.9572) (width 0.25) (layer B.Cu) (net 13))
 (segment (start 162 114.9572) (end 162 114.7572) (width 0.25) (layer B.Cu) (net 13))
 (segment (start 162 116.967) (end 162 117.967) (width 0.25) (layer B.Cu) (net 14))
 (segment (start 162 117.967) (end 162.78301 118.75001) (width 0.25) (layer B.Cu) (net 14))
 (segment (start 168.5344 115.0954) (end 169.4844 115.0954) (width 0.25) (layer B.Cu) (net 14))
 (segment (start 162.78301 118.75001) (end 167.044978 118.75001) (width 0.25) (layer B.Cu) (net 14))
 (segment (start 167.044978 118.75001) (end 167.877199 117.917789) (width 0.25) (layer B.Cu) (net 14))
 (segment (start 167.877199 115.752601) (end 168.5344 115.0954) (width 0.25) (layer B.Cu) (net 14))
 (segment (start 167.877199 117.917789) (end 167.877199 115.752601) (width 0.25) (layer B.Cu) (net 14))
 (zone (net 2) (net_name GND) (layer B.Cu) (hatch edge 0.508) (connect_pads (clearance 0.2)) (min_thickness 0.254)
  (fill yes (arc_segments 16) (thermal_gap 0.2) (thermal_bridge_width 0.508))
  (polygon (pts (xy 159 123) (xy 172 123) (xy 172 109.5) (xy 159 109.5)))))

